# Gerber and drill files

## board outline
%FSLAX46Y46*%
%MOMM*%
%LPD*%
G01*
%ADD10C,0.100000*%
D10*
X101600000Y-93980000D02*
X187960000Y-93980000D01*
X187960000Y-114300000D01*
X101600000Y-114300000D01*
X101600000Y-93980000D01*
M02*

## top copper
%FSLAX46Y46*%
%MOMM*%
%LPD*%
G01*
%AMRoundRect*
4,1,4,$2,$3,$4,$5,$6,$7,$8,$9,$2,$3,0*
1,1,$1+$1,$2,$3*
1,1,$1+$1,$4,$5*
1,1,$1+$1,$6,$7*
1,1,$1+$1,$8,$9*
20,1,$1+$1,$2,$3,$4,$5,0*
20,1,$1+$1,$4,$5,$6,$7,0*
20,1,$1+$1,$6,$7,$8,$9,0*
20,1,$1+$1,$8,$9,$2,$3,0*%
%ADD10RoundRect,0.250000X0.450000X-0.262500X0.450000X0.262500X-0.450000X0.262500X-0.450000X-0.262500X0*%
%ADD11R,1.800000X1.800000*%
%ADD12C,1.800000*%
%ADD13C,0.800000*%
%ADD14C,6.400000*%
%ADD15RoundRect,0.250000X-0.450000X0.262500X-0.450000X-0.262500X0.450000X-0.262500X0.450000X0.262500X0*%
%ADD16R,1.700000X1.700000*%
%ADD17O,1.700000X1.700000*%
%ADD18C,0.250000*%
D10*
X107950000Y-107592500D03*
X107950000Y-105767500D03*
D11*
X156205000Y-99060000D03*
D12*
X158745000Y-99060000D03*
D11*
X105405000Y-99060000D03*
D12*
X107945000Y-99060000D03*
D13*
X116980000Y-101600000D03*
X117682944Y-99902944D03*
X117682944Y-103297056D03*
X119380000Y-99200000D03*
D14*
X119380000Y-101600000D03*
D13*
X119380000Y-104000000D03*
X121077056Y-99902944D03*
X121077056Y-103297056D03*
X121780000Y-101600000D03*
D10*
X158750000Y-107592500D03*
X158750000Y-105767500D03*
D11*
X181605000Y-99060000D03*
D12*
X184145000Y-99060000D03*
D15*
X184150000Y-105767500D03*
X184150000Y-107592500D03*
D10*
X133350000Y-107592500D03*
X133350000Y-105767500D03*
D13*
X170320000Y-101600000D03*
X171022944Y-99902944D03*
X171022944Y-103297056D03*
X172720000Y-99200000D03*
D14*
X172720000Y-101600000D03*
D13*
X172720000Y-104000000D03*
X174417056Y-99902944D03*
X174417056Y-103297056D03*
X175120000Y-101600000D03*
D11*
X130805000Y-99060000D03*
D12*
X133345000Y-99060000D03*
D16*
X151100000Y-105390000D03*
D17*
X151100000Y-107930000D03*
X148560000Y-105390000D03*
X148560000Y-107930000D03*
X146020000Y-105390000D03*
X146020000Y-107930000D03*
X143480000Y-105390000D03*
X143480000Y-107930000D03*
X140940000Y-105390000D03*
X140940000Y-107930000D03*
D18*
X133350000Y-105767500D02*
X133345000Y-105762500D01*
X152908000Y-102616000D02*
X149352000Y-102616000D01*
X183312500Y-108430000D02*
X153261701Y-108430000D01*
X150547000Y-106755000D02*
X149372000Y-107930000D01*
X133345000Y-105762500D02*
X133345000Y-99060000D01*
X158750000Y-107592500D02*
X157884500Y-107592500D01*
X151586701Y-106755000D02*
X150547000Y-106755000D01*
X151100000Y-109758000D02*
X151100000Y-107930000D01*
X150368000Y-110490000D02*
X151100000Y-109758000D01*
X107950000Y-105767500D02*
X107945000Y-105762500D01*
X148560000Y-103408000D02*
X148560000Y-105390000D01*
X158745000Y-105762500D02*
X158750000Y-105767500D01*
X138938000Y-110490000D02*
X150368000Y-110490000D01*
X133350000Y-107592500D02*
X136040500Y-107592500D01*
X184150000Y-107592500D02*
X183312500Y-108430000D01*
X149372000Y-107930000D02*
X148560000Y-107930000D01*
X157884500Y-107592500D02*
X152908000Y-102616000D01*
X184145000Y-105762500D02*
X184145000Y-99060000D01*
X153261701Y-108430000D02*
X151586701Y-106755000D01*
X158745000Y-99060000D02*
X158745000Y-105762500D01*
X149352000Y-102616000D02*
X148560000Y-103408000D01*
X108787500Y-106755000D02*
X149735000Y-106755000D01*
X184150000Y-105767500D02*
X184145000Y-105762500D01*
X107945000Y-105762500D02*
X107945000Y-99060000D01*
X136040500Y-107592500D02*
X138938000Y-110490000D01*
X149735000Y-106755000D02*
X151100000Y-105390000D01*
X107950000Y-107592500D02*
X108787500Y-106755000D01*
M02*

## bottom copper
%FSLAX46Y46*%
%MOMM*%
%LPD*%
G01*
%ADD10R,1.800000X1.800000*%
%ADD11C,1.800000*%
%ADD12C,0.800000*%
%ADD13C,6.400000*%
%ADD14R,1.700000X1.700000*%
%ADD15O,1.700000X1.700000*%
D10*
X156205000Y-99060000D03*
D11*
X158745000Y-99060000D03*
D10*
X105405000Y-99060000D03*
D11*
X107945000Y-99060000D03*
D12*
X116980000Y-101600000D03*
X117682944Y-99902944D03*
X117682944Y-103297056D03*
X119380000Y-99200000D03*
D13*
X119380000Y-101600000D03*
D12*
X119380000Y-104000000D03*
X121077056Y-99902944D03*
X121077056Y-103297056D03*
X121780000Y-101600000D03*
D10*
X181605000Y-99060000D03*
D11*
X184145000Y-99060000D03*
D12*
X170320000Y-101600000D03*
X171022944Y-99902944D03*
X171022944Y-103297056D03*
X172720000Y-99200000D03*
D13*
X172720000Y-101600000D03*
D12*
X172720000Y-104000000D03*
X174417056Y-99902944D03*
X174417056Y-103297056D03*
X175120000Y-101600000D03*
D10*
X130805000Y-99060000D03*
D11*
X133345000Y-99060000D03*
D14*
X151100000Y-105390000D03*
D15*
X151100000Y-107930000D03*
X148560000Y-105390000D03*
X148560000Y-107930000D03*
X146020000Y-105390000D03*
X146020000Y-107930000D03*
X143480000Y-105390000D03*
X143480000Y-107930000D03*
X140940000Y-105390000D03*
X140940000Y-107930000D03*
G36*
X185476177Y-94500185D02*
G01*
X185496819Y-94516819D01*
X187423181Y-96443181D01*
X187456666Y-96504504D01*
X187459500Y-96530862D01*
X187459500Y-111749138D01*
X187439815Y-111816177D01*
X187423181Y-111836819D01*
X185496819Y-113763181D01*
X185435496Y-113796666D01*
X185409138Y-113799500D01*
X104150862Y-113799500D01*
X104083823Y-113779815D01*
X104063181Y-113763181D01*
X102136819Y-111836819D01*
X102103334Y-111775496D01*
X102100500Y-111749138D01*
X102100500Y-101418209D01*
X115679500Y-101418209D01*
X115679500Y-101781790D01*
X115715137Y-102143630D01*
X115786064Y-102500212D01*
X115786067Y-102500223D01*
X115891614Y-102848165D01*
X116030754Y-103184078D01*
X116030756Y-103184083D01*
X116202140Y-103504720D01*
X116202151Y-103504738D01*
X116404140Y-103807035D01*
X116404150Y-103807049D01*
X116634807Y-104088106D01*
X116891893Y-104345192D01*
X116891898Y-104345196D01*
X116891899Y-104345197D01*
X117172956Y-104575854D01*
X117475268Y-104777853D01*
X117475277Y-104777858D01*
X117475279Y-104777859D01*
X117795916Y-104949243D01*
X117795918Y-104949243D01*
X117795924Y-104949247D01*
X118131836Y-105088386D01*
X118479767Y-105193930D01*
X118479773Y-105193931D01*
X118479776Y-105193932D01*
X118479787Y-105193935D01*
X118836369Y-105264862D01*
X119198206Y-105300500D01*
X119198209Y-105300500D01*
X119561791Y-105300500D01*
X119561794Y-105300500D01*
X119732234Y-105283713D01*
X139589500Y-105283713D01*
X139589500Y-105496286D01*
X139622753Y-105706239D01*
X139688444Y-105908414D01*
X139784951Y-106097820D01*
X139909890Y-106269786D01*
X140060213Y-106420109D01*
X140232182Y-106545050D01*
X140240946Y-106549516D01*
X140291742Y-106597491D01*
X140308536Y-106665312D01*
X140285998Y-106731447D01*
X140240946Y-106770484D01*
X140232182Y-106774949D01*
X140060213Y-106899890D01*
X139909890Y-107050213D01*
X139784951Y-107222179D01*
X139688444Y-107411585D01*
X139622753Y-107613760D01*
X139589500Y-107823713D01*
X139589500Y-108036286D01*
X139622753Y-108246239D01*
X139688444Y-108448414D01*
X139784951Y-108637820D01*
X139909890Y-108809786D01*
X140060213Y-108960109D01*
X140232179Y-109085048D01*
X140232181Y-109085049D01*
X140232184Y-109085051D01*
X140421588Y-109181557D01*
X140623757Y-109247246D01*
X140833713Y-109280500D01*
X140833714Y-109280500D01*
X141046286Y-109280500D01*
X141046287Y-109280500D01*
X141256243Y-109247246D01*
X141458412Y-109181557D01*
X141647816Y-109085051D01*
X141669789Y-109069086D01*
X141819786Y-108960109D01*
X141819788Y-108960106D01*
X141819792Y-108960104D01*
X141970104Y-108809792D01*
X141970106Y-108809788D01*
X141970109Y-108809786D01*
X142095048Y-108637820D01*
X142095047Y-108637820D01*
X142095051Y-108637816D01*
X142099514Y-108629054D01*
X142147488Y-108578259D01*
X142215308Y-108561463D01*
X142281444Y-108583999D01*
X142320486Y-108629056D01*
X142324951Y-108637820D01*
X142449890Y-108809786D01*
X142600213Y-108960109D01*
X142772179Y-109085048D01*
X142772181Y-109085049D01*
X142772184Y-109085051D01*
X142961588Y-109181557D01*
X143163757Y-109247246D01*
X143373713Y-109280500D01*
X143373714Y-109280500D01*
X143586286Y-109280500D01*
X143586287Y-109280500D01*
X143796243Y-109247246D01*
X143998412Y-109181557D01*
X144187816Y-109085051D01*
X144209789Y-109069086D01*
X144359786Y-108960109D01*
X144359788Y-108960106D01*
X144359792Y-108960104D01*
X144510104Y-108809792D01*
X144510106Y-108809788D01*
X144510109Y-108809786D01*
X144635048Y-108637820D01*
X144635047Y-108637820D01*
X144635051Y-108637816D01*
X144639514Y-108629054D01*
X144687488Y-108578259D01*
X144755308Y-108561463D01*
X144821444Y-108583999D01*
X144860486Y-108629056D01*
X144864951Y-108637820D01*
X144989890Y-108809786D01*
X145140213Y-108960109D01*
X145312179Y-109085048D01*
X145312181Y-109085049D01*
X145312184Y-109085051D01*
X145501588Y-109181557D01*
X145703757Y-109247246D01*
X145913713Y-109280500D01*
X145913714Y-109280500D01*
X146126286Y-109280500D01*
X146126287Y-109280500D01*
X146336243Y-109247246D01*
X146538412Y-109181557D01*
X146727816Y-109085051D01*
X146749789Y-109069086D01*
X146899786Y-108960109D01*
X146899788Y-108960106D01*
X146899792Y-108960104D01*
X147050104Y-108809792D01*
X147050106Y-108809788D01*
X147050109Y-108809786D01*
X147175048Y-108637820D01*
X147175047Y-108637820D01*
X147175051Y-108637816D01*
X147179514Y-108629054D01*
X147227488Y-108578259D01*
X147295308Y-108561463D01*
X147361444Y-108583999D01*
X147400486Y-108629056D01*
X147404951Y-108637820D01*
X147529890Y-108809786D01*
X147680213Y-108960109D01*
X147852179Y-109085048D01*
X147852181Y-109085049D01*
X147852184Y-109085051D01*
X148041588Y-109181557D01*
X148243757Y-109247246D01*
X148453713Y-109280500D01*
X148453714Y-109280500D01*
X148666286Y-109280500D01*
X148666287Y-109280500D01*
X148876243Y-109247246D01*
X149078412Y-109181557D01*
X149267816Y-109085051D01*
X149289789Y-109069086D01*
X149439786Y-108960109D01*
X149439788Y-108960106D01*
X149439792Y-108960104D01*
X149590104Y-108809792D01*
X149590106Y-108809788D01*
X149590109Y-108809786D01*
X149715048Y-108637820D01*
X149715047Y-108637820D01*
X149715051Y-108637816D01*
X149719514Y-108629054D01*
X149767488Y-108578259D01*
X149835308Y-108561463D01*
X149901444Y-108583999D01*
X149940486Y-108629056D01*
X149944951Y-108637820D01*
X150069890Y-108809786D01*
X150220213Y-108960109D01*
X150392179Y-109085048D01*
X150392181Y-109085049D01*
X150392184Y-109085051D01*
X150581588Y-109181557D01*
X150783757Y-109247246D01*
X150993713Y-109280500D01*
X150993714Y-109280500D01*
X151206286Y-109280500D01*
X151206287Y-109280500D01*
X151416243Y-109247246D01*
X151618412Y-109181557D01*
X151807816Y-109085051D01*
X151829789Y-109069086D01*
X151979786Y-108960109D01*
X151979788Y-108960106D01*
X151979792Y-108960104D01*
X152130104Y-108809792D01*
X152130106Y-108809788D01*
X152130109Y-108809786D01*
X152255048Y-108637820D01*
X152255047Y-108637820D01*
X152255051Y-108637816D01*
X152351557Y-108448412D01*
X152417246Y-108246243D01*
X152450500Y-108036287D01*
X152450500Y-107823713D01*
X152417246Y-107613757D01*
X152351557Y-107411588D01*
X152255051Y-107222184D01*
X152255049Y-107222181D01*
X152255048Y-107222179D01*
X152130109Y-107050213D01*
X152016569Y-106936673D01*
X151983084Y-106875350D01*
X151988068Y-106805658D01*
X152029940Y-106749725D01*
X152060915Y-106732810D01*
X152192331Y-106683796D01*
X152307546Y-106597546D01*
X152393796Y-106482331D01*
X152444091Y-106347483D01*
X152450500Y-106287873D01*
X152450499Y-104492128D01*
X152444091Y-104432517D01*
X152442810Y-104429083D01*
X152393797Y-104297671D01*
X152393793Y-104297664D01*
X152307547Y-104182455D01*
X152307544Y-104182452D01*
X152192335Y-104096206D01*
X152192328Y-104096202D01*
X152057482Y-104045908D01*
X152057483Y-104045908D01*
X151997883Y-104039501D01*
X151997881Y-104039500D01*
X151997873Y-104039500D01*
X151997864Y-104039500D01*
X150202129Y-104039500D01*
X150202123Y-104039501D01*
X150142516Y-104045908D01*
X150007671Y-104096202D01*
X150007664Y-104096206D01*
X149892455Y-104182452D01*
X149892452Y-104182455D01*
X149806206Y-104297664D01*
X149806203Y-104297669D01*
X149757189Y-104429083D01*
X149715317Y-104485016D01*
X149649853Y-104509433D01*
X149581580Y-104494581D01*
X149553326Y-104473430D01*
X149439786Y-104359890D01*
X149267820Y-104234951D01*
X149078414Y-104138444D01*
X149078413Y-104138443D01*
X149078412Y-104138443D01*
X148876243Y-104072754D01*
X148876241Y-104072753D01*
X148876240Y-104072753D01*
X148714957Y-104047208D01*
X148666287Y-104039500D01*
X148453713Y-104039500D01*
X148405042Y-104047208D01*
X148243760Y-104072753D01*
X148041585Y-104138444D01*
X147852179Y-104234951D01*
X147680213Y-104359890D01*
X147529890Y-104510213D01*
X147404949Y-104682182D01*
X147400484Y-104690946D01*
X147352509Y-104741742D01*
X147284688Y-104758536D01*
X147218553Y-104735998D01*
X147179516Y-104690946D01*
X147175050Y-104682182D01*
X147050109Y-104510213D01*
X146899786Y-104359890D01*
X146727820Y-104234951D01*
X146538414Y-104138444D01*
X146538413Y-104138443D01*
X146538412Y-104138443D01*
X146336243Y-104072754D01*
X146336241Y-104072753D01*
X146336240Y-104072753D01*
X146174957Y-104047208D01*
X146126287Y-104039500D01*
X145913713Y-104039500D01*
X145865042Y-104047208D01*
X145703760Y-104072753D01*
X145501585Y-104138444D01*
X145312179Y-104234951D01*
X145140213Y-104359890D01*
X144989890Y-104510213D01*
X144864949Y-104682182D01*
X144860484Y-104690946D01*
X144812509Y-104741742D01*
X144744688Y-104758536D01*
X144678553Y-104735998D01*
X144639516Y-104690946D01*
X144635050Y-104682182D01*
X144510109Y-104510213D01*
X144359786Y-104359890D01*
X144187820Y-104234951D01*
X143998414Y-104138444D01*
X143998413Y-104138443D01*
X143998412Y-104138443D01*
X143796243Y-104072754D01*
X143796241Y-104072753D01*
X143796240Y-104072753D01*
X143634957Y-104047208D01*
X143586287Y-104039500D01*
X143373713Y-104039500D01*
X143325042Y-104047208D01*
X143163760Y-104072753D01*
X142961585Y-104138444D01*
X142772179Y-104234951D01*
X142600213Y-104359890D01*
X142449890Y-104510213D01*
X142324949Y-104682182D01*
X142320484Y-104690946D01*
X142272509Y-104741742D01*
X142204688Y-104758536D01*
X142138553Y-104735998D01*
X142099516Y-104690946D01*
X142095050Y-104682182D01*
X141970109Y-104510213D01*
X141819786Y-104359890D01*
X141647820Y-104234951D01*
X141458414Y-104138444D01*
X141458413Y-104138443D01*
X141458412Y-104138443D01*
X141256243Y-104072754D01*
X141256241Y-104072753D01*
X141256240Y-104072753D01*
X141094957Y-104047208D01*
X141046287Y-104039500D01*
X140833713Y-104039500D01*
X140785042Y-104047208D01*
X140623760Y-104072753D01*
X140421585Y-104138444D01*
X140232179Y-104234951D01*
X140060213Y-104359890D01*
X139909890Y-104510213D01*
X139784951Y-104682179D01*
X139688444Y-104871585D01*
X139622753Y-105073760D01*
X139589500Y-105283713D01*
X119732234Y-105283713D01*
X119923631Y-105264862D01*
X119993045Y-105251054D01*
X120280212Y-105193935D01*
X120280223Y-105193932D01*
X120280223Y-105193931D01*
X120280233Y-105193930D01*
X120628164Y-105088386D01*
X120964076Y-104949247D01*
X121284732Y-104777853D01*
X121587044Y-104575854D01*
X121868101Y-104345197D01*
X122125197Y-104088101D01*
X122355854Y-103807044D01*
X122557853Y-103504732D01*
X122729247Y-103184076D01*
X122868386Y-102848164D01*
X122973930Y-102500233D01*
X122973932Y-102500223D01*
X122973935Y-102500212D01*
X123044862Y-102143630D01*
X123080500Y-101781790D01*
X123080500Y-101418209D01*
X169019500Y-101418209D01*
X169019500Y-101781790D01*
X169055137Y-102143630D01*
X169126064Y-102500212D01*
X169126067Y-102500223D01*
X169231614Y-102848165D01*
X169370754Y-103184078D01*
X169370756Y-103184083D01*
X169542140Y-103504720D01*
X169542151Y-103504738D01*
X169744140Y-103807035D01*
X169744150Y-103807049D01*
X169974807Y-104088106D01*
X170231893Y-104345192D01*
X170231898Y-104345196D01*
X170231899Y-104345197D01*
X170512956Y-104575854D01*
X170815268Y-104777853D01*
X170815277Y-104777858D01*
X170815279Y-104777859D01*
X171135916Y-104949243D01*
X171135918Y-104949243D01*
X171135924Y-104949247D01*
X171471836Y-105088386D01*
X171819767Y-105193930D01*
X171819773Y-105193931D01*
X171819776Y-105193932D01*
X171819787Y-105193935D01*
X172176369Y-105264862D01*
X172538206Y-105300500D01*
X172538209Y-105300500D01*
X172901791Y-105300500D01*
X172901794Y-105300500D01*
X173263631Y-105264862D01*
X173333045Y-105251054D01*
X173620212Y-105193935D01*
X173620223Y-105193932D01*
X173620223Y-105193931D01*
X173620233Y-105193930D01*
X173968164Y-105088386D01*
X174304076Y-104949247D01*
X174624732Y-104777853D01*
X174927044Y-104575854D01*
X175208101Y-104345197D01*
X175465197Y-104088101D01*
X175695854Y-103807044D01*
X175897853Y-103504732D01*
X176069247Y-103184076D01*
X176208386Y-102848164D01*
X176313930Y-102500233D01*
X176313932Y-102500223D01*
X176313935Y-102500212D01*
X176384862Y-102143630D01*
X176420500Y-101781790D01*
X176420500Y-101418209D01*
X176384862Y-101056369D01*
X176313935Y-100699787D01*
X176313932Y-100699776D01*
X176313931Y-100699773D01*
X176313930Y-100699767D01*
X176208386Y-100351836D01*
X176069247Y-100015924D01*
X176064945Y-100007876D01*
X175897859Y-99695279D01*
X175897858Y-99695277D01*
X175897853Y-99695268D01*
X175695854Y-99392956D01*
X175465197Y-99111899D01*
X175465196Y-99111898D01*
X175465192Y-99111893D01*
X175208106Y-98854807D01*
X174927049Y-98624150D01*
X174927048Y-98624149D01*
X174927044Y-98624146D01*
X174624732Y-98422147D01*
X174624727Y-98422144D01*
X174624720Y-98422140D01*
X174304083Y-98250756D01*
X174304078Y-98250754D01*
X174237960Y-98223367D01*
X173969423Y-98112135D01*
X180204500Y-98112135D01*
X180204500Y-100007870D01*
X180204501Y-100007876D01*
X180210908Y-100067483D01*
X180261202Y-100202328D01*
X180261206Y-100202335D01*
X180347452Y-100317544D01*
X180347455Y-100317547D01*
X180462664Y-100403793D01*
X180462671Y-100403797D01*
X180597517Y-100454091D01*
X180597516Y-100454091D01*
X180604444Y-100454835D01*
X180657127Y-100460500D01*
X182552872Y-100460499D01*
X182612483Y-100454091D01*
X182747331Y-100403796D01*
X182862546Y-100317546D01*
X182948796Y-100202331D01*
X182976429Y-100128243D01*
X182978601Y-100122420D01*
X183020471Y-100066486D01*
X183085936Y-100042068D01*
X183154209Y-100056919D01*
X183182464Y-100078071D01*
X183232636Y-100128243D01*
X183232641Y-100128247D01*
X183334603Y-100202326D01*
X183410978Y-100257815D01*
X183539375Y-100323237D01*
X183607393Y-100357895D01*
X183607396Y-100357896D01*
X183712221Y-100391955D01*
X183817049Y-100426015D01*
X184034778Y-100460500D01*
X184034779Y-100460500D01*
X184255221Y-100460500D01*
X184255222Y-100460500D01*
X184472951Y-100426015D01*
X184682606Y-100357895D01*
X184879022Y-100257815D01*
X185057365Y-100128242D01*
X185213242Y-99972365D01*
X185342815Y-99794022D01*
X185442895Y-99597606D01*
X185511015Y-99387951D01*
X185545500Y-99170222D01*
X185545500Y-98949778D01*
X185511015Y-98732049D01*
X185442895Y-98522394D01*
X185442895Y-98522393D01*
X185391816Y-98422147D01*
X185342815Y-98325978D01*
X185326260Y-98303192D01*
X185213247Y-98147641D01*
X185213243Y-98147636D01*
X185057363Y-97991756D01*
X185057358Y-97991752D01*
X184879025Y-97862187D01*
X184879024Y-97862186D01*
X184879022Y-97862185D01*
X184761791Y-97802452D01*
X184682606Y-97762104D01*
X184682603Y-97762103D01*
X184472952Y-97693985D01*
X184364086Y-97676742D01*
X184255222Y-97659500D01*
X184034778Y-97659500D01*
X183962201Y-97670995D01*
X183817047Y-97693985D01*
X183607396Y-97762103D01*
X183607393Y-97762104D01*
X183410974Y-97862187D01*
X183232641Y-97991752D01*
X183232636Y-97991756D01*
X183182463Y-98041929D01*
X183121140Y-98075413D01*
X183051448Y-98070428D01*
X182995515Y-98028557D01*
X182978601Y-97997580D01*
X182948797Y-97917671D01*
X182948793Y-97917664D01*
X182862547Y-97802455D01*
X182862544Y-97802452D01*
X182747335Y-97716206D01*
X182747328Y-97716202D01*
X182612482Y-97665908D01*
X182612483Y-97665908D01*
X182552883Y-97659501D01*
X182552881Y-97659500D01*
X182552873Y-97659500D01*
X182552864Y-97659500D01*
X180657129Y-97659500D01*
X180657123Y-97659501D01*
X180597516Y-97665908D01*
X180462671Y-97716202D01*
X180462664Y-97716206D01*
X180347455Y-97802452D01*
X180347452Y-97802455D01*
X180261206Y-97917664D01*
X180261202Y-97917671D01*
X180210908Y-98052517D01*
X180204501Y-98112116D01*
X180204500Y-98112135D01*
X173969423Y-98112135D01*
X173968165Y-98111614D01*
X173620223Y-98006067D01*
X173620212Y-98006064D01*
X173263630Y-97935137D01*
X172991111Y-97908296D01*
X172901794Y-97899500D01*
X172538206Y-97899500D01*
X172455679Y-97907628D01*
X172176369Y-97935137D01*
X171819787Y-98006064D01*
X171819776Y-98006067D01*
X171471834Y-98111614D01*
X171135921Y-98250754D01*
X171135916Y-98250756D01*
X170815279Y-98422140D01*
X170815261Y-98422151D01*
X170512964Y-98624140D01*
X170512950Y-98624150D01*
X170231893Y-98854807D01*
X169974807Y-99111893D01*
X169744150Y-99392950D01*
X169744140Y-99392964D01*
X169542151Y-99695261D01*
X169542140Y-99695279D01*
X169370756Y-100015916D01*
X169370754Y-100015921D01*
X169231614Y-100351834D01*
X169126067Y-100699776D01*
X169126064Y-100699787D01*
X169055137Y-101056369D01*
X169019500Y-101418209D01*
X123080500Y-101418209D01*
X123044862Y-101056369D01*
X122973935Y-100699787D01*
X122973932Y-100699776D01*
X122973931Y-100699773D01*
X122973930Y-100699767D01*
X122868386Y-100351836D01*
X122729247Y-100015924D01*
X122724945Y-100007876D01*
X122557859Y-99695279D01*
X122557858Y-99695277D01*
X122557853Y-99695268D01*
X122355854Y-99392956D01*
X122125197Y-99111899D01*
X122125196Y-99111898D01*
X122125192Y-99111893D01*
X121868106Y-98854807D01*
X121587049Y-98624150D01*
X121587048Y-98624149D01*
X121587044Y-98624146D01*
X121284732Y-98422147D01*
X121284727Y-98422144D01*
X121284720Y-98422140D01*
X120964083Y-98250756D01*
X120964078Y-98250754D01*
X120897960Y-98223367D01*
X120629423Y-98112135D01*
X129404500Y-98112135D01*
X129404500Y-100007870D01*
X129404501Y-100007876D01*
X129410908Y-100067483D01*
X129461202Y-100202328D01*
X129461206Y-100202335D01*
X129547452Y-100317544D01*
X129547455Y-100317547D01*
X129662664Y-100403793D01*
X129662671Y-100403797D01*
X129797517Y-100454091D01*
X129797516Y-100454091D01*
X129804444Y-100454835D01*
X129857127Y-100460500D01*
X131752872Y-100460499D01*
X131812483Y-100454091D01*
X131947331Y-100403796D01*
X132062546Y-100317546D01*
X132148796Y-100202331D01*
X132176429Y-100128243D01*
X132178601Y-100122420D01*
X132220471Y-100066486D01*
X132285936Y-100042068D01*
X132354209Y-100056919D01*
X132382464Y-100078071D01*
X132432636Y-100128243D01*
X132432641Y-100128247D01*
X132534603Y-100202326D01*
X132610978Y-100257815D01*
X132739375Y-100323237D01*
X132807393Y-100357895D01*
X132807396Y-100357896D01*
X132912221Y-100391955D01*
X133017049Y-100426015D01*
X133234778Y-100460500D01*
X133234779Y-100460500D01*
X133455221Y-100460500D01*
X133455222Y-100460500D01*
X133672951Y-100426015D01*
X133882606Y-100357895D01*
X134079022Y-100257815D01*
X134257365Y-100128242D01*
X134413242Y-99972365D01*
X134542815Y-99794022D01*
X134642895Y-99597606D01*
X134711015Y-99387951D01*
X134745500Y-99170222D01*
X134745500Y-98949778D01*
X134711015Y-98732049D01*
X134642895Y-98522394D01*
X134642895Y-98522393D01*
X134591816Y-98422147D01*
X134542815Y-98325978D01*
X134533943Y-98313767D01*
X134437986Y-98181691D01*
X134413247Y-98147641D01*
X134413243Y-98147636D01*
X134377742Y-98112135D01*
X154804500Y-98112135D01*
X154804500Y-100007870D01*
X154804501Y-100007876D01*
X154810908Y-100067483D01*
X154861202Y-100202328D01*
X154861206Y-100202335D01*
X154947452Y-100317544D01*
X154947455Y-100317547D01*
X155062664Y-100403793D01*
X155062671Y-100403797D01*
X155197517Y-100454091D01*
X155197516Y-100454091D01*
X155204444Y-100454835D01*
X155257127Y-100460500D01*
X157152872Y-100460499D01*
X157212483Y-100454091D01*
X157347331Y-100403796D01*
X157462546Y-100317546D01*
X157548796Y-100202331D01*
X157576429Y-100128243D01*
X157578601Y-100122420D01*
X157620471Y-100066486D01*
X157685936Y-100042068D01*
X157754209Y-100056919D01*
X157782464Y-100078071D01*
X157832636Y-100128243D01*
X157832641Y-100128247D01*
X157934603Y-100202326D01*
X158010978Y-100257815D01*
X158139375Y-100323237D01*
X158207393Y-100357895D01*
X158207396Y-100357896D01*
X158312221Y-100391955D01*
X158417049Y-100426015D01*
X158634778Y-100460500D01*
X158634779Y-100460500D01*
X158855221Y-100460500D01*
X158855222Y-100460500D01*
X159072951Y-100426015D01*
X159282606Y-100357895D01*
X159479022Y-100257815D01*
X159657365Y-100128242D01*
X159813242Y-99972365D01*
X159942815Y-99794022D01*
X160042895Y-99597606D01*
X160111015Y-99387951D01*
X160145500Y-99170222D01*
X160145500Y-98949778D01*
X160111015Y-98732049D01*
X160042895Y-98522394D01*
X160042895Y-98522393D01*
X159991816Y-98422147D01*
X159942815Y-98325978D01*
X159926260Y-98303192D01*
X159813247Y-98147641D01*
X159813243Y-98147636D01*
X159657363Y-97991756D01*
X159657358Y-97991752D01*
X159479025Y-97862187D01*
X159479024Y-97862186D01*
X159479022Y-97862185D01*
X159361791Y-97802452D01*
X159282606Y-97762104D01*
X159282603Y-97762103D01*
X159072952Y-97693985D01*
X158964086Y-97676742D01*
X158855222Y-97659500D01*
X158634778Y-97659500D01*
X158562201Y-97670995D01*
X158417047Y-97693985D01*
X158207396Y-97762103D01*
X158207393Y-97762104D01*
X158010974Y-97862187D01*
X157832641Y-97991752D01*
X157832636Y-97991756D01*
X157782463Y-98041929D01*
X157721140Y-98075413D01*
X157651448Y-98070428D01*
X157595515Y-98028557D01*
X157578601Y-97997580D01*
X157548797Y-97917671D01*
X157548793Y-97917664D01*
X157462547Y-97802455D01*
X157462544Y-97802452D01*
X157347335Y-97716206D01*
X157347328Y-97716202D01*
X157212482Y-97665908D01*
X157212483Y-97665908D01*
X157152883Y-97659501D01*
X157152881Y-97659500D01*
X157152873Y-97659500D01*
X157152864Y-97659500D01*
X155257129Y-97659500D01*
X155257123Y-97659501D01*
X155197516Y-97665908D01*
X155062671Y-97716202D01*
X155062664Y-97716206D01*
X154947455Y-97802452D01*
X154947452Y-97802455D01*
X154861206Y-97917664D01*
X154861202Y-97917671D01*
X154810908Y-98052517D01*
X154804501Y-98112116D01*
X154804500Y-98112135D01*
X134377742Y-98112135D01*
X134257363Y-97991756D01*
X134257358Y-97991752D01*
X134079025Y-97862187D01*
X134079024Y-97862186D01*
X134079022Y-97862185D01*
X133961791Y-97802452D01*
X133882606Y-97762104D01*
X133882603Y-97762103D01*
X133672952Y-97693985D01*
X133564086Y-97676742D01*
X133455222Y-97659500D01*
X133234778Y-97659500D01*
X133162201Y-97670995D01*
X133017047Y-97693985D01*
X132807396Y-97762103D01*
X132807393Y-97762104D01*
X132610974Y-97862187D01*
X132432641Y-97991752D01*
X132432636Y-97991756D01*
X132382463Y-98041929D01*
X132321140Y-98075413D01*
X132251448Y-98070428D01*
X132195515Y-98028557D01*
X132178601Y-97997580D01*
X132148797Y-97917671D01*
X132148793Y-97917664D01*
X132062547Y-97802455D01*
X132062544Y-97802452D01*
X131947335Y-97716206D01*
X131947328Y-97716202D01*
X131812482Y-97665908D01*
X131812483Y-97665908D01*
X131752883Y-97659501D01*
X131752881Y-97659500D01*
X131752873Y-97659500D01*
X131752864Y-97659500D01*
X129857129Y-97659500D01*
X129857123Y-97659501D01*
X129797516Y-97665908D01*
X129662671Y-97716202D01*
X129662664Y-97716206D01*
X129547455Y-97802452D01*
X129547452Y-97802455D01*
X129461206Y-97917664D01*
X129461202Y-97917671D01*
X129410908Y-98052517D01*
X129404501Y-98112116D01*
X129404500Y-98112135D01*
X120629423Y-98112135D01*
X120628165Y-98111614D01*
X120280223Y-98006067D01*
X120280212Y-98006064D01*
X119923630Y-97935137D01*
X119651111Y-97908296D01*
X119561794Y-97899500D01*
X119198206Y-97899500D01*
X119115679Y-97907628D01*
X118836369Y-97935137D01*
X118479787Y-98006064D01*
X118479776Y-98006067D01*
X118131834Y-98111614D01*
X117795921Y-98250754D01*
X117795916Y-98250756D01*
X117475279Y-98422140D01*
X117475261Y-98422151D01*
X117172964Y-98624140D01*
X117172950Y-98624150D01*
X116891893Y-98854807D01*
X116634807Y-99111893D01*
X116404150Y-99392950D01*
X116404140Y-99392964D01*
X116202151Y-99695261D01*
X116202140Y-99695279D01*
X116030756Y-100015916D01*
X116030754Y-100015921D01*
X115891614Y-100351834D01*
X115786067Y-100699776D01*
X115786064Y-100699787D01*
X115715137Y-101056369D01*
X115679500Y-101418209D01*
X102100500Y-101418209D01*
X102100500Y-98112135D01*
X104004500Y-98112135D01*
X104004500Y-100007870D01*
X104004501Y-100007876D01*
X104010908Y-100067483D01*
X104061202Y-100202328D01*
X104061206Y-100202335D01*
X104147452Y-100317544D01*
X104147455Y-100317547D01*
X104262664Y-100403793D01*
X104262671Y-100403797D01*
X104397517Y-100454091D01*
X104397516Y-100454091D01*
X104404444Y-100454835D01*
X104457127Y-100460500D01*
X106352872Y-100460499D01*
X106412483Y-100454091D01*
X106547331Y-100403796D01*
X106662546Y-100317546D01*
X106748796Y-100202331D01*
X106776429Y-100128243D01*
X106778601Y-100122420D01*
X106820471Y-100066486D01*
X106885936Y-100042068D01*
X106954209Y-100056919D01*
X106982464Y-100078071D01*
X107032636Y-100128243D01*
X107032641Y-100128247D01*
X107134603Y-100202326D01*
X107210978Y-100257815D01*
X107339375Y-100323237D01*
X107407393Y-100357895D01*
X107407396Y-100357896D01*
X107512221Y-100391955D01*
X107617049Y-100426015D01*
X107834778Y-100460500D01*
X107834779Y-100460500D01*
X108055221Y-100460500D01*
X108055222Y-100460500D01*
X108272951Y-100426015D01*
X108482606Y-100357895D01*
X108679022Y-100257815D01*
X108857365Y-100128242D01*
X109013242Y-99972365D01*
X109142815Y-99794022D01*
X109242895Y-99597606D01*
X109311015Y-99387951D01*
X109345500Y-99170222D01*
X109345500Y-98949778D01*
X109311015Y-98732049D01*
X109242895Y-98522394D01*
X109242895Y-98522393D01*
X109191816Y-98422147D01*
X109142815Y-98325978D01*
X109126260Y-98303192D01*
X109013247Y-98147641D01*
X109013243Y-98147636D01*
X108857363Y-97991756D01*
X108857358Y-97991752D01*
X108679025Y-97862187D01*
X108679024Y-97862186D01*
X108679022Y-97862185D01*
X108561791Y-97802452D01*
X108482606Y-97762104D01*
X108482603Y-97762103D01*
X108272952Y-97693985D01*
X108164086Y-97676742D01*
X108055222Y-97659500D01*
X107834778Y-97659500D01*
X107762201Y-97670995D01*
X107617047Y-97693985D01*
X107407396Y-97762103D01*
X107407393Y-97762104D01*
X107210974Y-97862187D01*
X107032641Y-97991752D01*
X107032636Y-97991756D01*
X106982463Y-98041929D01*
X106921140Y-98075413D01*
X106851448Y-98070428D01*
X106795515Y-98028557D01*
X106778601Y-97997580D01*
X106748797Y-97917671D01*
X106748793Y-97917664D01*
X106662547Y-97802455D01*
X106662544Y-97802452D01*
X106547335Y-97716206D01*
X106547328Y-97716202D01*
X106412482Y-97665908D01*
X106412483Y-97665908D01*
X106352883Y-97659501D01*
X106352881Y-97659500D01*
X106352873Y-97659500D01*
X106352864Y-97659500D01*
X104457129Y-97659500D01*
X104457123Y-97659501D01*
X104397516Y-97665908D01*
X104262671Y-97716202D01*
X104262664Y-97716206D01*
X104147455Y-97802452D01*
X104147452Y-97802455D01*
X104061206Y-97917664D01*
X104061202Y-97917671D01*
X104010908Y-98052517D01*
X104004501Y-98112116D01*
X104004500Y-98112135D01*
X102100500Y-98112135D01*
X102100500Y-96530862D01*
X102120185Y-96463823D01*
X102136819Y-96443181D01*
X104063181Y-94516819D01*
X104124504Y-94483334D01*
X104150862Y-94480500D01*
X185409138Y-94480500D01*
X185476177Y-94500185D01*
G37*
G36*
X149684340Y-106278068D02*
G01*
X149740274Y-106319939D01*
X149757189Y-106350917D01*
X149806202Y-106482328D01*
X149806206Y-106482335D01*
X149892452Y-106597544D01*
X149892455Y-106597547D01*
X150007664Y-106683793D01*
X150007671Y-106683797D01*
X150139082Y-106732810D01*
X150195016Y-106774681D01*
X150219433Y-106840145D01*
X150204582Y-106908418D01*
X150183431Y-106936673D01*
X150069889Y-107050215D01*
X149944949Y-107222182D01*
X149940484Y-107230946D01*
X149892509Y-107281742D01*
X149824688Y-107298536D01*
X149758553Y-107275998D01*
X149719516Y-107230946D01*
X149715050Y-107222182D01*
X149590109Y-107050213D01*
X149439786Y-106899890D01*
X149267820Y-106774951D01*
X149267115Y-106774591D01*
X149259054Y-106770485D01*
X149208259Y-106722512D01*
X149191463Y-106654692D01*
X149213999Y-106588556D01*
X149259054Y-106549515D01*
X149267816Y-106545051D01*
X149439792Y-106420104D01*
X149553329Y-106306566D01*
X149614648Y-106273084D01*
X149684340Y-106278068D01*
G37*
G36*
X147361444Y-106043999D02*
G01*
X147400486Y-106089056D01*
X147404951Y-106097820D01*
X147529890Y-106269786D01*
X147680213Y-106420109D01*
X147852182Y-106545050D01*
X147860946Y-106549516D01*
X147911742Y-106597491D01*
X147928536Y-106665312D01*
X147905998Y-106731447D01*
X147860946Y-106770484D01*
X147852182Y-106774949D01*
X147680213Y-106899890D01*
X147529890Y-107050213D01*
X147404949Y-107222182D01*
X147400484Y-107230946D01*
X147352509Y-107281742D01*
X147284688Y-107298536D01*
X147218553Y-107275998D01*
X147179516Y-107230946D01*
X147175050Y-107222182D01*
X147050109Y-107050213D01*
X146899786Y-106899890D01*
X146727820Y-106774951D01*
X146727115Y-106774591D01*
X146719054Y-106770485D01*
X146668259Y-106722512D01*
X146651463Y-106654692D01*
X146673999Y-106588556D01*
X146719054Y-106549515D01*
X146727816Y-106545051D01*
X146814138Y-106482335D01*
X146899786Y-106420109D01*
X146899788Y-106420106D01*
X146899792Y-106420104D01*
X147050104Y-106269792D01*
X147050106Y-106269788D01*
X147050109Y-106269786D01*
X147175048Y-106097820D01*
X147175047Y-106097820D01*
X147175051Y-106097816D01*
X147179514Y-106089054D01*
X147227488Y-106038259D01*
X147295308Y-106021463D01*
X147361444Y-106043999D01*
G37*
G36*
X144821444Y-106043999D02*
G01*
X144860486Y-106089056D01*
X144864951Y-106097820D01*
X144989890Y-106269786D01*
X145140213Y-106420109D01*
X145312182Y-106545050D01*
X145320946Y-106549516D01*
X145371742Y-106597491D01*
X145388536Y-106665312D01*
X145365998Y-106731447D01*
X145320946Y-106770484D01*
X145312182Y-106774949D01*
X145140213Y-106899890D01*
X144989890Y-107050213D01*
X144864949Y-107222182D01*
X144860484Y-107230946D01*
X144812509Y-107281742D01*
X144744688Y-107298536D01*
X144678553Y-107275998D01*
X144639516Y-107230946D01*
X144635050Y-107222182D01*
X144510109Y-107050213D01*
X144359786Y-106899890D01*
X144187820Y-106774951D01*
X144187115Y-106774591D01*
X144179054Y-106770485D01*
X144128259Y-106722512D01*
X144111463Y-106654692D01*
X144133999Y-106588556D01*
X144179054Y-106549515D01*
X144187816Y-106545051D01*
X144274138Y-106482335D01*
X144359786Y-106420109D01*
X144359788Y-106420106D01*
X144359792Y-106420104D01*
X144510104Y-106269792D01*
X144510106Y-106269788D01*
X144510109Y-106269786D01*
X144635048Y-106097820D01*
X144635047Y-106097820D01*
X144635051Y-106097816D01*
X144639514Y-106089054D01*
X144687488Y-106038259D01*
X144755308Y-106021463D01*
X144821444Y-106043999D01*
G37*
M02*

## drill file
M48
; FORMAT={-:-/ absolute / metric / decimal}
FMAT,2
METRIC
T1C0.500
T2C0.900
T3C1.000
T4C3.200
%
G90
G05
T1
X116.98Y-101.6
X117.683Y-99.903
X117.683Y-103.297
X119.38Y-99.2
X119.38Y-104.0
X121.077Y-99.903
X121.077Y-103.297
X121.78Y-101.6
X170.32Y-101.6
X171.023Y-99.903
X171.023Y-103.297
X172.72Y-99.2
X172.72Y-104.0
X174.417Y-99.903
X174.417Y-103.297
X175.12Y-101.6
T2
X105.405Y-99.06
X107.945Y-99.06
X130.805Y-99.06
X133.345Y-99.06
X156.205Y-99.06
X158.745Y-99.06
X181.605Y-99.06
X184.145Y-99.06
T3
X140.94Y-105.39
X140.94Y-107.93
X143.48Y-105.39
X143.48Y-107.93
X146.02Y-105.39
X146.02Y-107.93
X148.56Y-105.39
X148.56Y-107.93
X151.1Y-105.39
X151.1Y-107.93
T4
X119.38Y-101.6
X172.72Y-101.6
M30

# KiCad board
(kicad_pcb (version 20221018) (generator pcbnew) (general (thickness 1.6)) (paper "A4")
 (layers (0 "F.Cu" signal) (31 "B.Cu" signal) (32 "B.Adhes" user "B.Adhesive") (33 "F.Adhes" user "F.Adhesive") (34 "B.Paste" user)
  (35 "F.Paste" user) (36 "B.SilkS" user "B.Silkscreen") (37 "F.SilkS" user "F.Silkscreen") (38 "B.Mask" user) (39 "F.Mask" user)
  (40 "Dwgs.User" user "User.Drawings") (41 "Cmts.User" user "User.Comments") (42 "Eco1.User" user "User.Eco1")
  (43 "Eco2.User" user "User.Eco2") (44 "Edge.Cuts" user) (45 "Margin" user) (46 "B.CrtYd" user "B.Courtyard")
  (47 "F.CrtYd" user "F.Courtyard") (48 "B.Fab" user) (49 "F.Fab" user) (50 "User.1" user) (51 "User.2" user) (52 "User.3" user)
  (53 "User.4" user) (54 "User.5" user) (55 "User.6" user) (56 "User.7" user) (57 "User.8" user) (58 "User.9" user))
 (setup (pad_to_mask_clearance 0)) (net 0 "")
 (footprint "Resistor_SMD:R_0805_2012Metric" (layer "F.Cu") (at 107.95 106.68 90)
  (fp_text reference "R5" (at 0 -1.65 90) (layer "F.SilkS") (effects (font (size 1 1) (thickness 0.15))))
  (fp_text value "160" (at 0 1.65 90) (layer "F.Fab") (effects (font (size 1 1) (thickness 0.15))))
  (pad "1" smd roundrect (at -0.9125 0 90) (size 1.025 1.4) (layers "F.Cu" "F.Paste" "F.Mask") (roundrect_rratio 0.243902439))
  (pad "2" smd roundrect (at 0.9125 0 90) (size 1.025 1.4) (layers "F.Cu" "F.Paste" "F.Mask") (roundrect_rratio 0.243902439)))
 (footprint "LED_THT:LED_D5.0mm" (layer "F.Cu") (at 156.205 99.06)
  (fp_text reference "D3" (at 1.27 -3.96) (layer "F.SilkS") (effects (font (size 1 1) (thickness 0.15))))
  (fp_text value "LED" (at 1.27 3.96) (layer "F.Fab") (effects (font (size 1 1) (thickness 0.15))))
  (pad "1" thru_hole rect (at 0 0) (size 1.8 1.8) (drill 0.9) (layers "*.Cu" "*.Mask"))
  (pad "2" thru_hole circle (at 2.54 0) (size 1.8 1.8) (drill 0.9) (layers "*.Cu" "*.Mask")))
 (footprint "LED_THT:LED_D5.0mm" (layer "F.Cu") (at 105.405 99.06)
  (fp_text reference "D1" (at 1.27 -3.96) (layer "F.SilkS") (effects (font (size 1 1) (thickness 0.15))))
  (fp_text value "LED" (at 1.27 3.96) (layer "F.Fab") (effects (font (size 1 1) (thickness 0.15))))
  (pad "1" thru_hole rect (at 0 0) (size 1.8 1.8) (drill 0.9) (layers "*.Cu" "*.Mask"))
  (pad "2" thru_hole circle (at 2.54 0) (size 1.8 1.8) (drill 0.9) (layers "*.Cu" "*.Mask")))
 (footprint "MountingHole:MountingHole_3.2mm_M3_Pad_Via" (layer "F.Cu") (at 119.38 101.6)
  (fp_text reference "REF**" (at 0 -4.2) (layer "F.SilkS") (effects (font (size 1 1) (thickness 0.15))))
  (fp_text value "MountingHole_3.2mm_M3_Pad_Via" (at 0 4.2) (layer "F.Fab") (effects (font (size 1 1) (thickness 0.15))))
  (pad "1" thru_hole circle (at -2.4 0) (size 0.8 0.8) (drill 0.5) (layers "*.Cu" "*.Mask"))
  (pad "1" thru_hole circle (at -1.697056 -1.697056) (size 0.8 0.8) (drill 0.5) (layers "*.Cu" "*.Mask"))
  (pad "1" thru_hole circle (at -1.697056 1.697056) (size 0.8 0.8) (drill 0.5) (layers "*.Cu" "*.Mask"))
  (pad "1" thru_hole circle (at 0 -2.4) (size 0.8 0.8) (drill 0.5) (layers "*.Cu" "*.Mask"))
  (pad "1" thru_hole circle (at 0 0) (size 6.4 6.4) (drill 3.2) (layers "*.Cu" "*.Mask"))
  (pad "1" thru_hole circle (at 0 2.4) (size 0.8 0.8) (drill 0.5) (layers "*.Cu" "*.Mask"))
  (pad "1" thru_hole circle (at 1.697056 -1.697056) (size 0.8 0.8) (drill 0.5) (layers "*.Cu" "*.Mask"))
  (pad "1" thru_hole circle (at 1.697056 1.697056) (size 0.8 0.8) (drill 0.5) (layers "*.Cu" "*.Mask"))
  (pad "1" thru_hole circle (at 2.4 0) (size 0.8 0.8) (drill 0.5) (layers "*.Cu" "*.Mask")))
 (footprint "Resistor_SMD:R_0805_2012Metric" (layer "F.Cu") (at 158.75 106.68 90)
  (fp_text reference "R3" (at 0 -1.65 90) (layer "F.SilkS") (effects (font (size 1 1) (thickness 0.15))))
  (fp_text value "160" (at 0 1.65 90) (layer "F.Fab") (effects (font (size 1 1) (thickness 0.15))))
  (pad "1" smd roundrect (at -0.9125 0 90) (size 1.025 1.4) (layers "F.Cu" "F.Paste" "F.Mask") (roundrect_rratio 0.243902439))
  (pad "2" smd roundrect (at 0.9125 0 90) (size 1.025 1.4) (layers "F.Cu" "F.Paste" "F.Mask") (roundrect_rratio 0.243902439)))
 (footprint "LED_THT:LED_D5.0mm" (layer "F.Cu") (at 181.605 99.06)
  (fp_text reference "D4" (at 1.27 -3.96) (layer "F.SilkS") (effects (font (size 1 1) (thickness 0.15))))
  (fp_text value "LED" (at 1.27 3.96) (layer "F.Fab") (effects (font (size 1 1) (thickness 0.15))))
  (pad "1" thru_hole rect (at 0 0) (size 1.8 1.8) (drill 0.9) (layers "*.Cu" "*.Mask"))
  (pad "2" thru_hole circle (at 2.54 0) (size 1.8 1.8) (drill 0.9) (layers "*.Cu" "*.Mask")))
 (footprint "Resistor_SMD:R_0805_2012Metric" (layer "F.Cu") (at 184.15 106.68 -90)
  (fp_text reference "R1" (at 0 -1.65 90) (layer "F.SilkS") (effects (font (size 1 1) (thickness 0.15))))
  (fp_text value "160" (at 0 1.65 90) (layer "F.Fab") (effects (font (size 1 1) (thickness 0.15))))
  (pad "1" smd roundrect (at -0.9125 0 270) (size 1.025 1.4) (layers "F.Cu" "F.Paste" "F.Mask") (roundrect_rratio 0.243902439))
  (pad "2" smd roundrect (at 0.9125 0 270) (size 1.025 1.4) (layers "F.Cu" "F.Paste" "F.Mask") (roundrect_rratio 0.243902439)))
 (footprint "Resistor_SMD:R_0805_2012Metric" (layer "F.Cu") (at 133.35 106.68 90)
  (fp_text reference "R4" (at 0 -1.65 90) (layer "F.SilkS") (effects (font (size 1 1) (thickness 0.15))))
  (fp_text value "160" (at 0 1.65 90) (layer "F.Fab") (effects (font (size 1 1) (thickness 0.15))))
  (pad "1" smd roundrect (at -0.9125 0 90) (size 1.025 1.4) (layers "F.Cu" "F.Paste" "F.Mask") (roundrect_rratio 0.243902439))
  (pad "2" smd roundrect (at 0.9125 0 90) (size 1.025 1.4) (layers "F.Cu" "F.Paste" "F.Mask") (roundrect_rratio 0.243902439)))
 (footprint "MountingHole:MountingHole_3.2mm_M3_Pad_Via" (layer "F.Cu") (at 172.72 101.6)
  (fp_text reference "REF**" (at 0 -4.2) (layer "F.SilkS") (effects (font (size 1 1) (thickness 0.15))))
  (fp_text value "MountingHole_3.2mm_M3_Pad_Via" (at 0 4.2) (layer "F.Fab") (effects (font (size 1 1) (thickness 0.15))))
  (pad "1" thru_hole circle (at -2.4 0) (size 0.8 0.8) (drill 0.5) (layers "*.Cu" "*.Mask"))
  (pad "1" thru_hole circle (at -1.697056 -1.697056) (size 0.8 0.8) (drill 0.5) (layers "*.Cu" "*.Mask"))
  (pad "1" thru_hole circle (at -1.697056 1.697056) (size 0.8 0.8) (drill 0.5) (layers "*.Cu" "*.Mask"))
  (pad "1" thru_hole circle (at 0 -2.4) (size 0.8 0.8) (drill 0.5) (layers "*.Cu" "*.Mask"))
  (pad "1" thru_hole circle (at 0 0) (size 6.4 6.4) (drill 3.2) (layers "*.Cu" "*.Mask"))
  (pad "1" thru_hole circle (at 0 2.4) (size 0.8 0.8) (drill 0.5) (layers "*.Cu" "*.Mask"))
  (pad "1" thru_hole circle (at 1.697056 -1.697056) (size 0.8 0.8) (drill 0.5) (layers "*.Cu" "*.Mask"))
  (pad "1" thru_hole circle (at 1.697056 1.697056) (size 0.8 0.8) (drill 0.5) (layers "*.Cu" "*.Mask"))
  (pad "1" thru_hole circle (at 2.4 0) (size 0.8 0.8) (drill 0.5) (layers "*.Cu" "*.Mask")))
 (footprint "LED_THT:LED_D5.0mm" (layer "F.Cu") (at 130.805 99.06)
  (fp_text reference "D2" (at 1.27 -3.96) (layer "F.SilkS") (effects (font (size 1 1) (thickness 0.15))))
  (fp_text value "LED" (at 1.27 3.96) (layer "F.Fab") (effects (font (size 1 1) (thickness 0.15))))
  (pad "1" thru_hole rect (at 0 0) (size 1.8 1.8) (drill 0.9) (layers "*.Cu" "*.Mask"))
  (pad "2" thru_hole circle (at 2.54 0) (size 1.8 1.8) (drill 0.9) (layers "*.Cu" "*.Mask")))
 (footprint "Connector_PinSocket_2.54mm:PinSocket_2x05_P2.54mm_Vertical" (layer "B.Cu") (at 151.1 105.39 90)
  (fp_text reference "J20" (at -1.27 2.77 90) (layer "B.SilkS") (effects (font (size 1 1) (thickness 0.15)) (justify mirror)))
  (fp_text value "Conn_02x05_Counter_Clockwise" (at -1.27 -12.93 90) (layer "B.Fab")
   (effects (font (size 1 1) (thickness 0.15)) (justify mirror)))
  (pad "1" thru_hole rect (at 0 0 90) (size 1.7 1.7) (drill 1) (layers "*.Cu" "*.Mask"))
  (pad "2" thru_hole oval (at -2.54 0 90) (size 1.7 1.7) (drill 1) (layers "*.Cu" "*.Mask"))
  (pad "3" thru_hole oval (at 0 -2.54 90) (size 1.7 1.7) (drill 1) (layers "*.Cu" "*.Mask"))
  (pad "4" thru_hole oval (at -2.54 -2.54 90) (size 1.7 1.7) (drill 1) (layers "*.Cu" "*.Mask"))
  (pad "5" thru_hole oval (at 0 -5.08 90) (size 1.7 1.7) (drill 1) (layers "*.Cu" "*.Mask"))
  (pad "6" thru_hole oval (at -2.54 -5.08 90) (size 1.7 1.7) (drill 1) (layers "*.Cu" "*.Mask"))
  (pad "7" thru_hole oval (at 0 -7.62 90) (size 1.7 1.7) (drill 1) (layers "*.Cu" "*.Mask"))
  (pad "8" thru_hole oval (at -2.54 -7.62 90) (size 1.7 1.7) (drill 1) (layers "*.Cu" "*.Mask"))
  (pad "9" thru_hole oval (at 0 -10.16 90) (size 1.7 1.7) (drill 1) (layers "*.Cu" "*.Mask"))
  (pad "10" thru_hole oval (at -2.54 -10.16 90) (size 1.7 1.7) (drill 1) (layers "*.Cu" "*.Mask")))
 (gr_rect (start 101.6 93.98) (end 187.96 114.3) (stroke (width 0.1) (type default)) (fill none) (layer "Edge.Cuts"))
 (segment (start 133.35 105.7675) (end 133.345 105.7625) (width 0.25) (layer "F.Cu") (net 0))
 (segment (start 152.908 102.616) (end 149.352 102.616) (width 0.25) (layer "F.Cu") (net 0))
 (segment (start 183.3125 108.43) (end 153.261701 108.43) (width 0.25) (layer "F.Cu") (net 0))
 (segment (start 150.547 106.755) (end 149.372 107.93) (width 0.25) (layer "F.Cu") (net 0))
 (segment (start 133.345 105.7625) (end 133.345 99.06) (width 0.25) (layer "F.Cu") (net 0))
 (segment (start 158.75 107.5925) (end 157.8845 107.5925) (width 0.25) (layer "F.Cu") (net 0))
 (segment (start 151.586701 106.755) (end 150.547 106.755) (width 0.25) (layer "F.Cu") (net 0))
 (segment (start 151.1 109.758) (end 151.1 107.93) (width 0.25) (layer "F.Cu") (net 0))
 (segment (start 150.368 110.49) (end 151.1 109.758) (width 0.25) (layer "F.Cu") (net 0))
 (segment (start 107.95 105.7675) (end 107.945 105.7625) (width 0.25) (layer "F.Cu") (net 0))
 (segment (start 148.56 103.408) (end 148.56 105.39) (width 0.25) (layer "F.Cu") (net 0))
 (segment (start 158.745 105.7625) (end 158.75 105.7675) (width 0.25) (layer "F.Cu") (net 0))
 (segment (start 138.938 110.49) (end 150.368 110.49) (width 0.25) (layer "F.Cu") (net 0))
 (segment (start 133.35 107.5925) (end 136.0405 107.5925) (width 0.25) (layer "F.Cu") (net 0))
 (segment (start 184.15 107.5925) (end 183.3125 108.43) (width 0.25) (layer "F.Cu") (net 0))
 (segment (start 149.372 107.93) (end 148.56 107.93) (width 0.25) (layer "F.Cu") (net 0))
 (segment (start 157.8845 107.5925) (end 152.908 102.616) (width 0.25) (layer "F.Cu") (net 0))
 (segment (start 184.145 105.7625) (end 184.145 99.06) (width 0.25) (layer "F.Cu") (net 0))
 (segment (start 153.261701 108.43) (end 151.586701 106.755) (width 0.25) (layer "F.Cu") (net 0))
 (segment (start 158.745 99.06) (end 158.745 105.7625) (width 0.25) (layer "F.Cu") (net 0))
 (segment (start 149.352 102.616) (end 148.56 103.408) (width 0.25) (layer "F.Cu") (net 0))
 (segment (start 108.7875 106.755) (end 149.735 106.755) (width 0.25) (layer "F.Cu") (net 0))
 (segment (start 184.15 105.7675) (end 184.145 105.7625) (width 0.25) (layer "F.Cu") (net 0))
 (segment (start 107.945 105.7625) (end 107.945 99.06) (width 0.25) (layer "F.Cu") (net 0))
 (segment (start 136.0405 107.5925) (end 138.938 110.49) (width 0.25) (layer "F.Cu") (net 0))
 (segment (start 149.735 106.755) (end 151.1 105.39) (width 0.25) (layer "F.Cu") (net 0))
 (segment (start 107.95 107.5925) (end 108.7875 106.755) (width 0.25) (layer "F.Cu") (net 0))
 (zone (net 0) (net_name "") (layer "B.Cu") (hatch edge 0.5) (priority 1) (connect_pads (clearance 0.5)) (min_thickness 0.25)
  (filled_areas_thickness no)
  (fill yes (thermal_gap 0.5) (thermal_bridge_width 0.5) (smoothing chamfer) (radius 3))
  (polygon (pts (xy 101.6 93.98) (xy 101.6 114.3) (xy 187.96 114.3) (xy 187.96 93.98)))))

